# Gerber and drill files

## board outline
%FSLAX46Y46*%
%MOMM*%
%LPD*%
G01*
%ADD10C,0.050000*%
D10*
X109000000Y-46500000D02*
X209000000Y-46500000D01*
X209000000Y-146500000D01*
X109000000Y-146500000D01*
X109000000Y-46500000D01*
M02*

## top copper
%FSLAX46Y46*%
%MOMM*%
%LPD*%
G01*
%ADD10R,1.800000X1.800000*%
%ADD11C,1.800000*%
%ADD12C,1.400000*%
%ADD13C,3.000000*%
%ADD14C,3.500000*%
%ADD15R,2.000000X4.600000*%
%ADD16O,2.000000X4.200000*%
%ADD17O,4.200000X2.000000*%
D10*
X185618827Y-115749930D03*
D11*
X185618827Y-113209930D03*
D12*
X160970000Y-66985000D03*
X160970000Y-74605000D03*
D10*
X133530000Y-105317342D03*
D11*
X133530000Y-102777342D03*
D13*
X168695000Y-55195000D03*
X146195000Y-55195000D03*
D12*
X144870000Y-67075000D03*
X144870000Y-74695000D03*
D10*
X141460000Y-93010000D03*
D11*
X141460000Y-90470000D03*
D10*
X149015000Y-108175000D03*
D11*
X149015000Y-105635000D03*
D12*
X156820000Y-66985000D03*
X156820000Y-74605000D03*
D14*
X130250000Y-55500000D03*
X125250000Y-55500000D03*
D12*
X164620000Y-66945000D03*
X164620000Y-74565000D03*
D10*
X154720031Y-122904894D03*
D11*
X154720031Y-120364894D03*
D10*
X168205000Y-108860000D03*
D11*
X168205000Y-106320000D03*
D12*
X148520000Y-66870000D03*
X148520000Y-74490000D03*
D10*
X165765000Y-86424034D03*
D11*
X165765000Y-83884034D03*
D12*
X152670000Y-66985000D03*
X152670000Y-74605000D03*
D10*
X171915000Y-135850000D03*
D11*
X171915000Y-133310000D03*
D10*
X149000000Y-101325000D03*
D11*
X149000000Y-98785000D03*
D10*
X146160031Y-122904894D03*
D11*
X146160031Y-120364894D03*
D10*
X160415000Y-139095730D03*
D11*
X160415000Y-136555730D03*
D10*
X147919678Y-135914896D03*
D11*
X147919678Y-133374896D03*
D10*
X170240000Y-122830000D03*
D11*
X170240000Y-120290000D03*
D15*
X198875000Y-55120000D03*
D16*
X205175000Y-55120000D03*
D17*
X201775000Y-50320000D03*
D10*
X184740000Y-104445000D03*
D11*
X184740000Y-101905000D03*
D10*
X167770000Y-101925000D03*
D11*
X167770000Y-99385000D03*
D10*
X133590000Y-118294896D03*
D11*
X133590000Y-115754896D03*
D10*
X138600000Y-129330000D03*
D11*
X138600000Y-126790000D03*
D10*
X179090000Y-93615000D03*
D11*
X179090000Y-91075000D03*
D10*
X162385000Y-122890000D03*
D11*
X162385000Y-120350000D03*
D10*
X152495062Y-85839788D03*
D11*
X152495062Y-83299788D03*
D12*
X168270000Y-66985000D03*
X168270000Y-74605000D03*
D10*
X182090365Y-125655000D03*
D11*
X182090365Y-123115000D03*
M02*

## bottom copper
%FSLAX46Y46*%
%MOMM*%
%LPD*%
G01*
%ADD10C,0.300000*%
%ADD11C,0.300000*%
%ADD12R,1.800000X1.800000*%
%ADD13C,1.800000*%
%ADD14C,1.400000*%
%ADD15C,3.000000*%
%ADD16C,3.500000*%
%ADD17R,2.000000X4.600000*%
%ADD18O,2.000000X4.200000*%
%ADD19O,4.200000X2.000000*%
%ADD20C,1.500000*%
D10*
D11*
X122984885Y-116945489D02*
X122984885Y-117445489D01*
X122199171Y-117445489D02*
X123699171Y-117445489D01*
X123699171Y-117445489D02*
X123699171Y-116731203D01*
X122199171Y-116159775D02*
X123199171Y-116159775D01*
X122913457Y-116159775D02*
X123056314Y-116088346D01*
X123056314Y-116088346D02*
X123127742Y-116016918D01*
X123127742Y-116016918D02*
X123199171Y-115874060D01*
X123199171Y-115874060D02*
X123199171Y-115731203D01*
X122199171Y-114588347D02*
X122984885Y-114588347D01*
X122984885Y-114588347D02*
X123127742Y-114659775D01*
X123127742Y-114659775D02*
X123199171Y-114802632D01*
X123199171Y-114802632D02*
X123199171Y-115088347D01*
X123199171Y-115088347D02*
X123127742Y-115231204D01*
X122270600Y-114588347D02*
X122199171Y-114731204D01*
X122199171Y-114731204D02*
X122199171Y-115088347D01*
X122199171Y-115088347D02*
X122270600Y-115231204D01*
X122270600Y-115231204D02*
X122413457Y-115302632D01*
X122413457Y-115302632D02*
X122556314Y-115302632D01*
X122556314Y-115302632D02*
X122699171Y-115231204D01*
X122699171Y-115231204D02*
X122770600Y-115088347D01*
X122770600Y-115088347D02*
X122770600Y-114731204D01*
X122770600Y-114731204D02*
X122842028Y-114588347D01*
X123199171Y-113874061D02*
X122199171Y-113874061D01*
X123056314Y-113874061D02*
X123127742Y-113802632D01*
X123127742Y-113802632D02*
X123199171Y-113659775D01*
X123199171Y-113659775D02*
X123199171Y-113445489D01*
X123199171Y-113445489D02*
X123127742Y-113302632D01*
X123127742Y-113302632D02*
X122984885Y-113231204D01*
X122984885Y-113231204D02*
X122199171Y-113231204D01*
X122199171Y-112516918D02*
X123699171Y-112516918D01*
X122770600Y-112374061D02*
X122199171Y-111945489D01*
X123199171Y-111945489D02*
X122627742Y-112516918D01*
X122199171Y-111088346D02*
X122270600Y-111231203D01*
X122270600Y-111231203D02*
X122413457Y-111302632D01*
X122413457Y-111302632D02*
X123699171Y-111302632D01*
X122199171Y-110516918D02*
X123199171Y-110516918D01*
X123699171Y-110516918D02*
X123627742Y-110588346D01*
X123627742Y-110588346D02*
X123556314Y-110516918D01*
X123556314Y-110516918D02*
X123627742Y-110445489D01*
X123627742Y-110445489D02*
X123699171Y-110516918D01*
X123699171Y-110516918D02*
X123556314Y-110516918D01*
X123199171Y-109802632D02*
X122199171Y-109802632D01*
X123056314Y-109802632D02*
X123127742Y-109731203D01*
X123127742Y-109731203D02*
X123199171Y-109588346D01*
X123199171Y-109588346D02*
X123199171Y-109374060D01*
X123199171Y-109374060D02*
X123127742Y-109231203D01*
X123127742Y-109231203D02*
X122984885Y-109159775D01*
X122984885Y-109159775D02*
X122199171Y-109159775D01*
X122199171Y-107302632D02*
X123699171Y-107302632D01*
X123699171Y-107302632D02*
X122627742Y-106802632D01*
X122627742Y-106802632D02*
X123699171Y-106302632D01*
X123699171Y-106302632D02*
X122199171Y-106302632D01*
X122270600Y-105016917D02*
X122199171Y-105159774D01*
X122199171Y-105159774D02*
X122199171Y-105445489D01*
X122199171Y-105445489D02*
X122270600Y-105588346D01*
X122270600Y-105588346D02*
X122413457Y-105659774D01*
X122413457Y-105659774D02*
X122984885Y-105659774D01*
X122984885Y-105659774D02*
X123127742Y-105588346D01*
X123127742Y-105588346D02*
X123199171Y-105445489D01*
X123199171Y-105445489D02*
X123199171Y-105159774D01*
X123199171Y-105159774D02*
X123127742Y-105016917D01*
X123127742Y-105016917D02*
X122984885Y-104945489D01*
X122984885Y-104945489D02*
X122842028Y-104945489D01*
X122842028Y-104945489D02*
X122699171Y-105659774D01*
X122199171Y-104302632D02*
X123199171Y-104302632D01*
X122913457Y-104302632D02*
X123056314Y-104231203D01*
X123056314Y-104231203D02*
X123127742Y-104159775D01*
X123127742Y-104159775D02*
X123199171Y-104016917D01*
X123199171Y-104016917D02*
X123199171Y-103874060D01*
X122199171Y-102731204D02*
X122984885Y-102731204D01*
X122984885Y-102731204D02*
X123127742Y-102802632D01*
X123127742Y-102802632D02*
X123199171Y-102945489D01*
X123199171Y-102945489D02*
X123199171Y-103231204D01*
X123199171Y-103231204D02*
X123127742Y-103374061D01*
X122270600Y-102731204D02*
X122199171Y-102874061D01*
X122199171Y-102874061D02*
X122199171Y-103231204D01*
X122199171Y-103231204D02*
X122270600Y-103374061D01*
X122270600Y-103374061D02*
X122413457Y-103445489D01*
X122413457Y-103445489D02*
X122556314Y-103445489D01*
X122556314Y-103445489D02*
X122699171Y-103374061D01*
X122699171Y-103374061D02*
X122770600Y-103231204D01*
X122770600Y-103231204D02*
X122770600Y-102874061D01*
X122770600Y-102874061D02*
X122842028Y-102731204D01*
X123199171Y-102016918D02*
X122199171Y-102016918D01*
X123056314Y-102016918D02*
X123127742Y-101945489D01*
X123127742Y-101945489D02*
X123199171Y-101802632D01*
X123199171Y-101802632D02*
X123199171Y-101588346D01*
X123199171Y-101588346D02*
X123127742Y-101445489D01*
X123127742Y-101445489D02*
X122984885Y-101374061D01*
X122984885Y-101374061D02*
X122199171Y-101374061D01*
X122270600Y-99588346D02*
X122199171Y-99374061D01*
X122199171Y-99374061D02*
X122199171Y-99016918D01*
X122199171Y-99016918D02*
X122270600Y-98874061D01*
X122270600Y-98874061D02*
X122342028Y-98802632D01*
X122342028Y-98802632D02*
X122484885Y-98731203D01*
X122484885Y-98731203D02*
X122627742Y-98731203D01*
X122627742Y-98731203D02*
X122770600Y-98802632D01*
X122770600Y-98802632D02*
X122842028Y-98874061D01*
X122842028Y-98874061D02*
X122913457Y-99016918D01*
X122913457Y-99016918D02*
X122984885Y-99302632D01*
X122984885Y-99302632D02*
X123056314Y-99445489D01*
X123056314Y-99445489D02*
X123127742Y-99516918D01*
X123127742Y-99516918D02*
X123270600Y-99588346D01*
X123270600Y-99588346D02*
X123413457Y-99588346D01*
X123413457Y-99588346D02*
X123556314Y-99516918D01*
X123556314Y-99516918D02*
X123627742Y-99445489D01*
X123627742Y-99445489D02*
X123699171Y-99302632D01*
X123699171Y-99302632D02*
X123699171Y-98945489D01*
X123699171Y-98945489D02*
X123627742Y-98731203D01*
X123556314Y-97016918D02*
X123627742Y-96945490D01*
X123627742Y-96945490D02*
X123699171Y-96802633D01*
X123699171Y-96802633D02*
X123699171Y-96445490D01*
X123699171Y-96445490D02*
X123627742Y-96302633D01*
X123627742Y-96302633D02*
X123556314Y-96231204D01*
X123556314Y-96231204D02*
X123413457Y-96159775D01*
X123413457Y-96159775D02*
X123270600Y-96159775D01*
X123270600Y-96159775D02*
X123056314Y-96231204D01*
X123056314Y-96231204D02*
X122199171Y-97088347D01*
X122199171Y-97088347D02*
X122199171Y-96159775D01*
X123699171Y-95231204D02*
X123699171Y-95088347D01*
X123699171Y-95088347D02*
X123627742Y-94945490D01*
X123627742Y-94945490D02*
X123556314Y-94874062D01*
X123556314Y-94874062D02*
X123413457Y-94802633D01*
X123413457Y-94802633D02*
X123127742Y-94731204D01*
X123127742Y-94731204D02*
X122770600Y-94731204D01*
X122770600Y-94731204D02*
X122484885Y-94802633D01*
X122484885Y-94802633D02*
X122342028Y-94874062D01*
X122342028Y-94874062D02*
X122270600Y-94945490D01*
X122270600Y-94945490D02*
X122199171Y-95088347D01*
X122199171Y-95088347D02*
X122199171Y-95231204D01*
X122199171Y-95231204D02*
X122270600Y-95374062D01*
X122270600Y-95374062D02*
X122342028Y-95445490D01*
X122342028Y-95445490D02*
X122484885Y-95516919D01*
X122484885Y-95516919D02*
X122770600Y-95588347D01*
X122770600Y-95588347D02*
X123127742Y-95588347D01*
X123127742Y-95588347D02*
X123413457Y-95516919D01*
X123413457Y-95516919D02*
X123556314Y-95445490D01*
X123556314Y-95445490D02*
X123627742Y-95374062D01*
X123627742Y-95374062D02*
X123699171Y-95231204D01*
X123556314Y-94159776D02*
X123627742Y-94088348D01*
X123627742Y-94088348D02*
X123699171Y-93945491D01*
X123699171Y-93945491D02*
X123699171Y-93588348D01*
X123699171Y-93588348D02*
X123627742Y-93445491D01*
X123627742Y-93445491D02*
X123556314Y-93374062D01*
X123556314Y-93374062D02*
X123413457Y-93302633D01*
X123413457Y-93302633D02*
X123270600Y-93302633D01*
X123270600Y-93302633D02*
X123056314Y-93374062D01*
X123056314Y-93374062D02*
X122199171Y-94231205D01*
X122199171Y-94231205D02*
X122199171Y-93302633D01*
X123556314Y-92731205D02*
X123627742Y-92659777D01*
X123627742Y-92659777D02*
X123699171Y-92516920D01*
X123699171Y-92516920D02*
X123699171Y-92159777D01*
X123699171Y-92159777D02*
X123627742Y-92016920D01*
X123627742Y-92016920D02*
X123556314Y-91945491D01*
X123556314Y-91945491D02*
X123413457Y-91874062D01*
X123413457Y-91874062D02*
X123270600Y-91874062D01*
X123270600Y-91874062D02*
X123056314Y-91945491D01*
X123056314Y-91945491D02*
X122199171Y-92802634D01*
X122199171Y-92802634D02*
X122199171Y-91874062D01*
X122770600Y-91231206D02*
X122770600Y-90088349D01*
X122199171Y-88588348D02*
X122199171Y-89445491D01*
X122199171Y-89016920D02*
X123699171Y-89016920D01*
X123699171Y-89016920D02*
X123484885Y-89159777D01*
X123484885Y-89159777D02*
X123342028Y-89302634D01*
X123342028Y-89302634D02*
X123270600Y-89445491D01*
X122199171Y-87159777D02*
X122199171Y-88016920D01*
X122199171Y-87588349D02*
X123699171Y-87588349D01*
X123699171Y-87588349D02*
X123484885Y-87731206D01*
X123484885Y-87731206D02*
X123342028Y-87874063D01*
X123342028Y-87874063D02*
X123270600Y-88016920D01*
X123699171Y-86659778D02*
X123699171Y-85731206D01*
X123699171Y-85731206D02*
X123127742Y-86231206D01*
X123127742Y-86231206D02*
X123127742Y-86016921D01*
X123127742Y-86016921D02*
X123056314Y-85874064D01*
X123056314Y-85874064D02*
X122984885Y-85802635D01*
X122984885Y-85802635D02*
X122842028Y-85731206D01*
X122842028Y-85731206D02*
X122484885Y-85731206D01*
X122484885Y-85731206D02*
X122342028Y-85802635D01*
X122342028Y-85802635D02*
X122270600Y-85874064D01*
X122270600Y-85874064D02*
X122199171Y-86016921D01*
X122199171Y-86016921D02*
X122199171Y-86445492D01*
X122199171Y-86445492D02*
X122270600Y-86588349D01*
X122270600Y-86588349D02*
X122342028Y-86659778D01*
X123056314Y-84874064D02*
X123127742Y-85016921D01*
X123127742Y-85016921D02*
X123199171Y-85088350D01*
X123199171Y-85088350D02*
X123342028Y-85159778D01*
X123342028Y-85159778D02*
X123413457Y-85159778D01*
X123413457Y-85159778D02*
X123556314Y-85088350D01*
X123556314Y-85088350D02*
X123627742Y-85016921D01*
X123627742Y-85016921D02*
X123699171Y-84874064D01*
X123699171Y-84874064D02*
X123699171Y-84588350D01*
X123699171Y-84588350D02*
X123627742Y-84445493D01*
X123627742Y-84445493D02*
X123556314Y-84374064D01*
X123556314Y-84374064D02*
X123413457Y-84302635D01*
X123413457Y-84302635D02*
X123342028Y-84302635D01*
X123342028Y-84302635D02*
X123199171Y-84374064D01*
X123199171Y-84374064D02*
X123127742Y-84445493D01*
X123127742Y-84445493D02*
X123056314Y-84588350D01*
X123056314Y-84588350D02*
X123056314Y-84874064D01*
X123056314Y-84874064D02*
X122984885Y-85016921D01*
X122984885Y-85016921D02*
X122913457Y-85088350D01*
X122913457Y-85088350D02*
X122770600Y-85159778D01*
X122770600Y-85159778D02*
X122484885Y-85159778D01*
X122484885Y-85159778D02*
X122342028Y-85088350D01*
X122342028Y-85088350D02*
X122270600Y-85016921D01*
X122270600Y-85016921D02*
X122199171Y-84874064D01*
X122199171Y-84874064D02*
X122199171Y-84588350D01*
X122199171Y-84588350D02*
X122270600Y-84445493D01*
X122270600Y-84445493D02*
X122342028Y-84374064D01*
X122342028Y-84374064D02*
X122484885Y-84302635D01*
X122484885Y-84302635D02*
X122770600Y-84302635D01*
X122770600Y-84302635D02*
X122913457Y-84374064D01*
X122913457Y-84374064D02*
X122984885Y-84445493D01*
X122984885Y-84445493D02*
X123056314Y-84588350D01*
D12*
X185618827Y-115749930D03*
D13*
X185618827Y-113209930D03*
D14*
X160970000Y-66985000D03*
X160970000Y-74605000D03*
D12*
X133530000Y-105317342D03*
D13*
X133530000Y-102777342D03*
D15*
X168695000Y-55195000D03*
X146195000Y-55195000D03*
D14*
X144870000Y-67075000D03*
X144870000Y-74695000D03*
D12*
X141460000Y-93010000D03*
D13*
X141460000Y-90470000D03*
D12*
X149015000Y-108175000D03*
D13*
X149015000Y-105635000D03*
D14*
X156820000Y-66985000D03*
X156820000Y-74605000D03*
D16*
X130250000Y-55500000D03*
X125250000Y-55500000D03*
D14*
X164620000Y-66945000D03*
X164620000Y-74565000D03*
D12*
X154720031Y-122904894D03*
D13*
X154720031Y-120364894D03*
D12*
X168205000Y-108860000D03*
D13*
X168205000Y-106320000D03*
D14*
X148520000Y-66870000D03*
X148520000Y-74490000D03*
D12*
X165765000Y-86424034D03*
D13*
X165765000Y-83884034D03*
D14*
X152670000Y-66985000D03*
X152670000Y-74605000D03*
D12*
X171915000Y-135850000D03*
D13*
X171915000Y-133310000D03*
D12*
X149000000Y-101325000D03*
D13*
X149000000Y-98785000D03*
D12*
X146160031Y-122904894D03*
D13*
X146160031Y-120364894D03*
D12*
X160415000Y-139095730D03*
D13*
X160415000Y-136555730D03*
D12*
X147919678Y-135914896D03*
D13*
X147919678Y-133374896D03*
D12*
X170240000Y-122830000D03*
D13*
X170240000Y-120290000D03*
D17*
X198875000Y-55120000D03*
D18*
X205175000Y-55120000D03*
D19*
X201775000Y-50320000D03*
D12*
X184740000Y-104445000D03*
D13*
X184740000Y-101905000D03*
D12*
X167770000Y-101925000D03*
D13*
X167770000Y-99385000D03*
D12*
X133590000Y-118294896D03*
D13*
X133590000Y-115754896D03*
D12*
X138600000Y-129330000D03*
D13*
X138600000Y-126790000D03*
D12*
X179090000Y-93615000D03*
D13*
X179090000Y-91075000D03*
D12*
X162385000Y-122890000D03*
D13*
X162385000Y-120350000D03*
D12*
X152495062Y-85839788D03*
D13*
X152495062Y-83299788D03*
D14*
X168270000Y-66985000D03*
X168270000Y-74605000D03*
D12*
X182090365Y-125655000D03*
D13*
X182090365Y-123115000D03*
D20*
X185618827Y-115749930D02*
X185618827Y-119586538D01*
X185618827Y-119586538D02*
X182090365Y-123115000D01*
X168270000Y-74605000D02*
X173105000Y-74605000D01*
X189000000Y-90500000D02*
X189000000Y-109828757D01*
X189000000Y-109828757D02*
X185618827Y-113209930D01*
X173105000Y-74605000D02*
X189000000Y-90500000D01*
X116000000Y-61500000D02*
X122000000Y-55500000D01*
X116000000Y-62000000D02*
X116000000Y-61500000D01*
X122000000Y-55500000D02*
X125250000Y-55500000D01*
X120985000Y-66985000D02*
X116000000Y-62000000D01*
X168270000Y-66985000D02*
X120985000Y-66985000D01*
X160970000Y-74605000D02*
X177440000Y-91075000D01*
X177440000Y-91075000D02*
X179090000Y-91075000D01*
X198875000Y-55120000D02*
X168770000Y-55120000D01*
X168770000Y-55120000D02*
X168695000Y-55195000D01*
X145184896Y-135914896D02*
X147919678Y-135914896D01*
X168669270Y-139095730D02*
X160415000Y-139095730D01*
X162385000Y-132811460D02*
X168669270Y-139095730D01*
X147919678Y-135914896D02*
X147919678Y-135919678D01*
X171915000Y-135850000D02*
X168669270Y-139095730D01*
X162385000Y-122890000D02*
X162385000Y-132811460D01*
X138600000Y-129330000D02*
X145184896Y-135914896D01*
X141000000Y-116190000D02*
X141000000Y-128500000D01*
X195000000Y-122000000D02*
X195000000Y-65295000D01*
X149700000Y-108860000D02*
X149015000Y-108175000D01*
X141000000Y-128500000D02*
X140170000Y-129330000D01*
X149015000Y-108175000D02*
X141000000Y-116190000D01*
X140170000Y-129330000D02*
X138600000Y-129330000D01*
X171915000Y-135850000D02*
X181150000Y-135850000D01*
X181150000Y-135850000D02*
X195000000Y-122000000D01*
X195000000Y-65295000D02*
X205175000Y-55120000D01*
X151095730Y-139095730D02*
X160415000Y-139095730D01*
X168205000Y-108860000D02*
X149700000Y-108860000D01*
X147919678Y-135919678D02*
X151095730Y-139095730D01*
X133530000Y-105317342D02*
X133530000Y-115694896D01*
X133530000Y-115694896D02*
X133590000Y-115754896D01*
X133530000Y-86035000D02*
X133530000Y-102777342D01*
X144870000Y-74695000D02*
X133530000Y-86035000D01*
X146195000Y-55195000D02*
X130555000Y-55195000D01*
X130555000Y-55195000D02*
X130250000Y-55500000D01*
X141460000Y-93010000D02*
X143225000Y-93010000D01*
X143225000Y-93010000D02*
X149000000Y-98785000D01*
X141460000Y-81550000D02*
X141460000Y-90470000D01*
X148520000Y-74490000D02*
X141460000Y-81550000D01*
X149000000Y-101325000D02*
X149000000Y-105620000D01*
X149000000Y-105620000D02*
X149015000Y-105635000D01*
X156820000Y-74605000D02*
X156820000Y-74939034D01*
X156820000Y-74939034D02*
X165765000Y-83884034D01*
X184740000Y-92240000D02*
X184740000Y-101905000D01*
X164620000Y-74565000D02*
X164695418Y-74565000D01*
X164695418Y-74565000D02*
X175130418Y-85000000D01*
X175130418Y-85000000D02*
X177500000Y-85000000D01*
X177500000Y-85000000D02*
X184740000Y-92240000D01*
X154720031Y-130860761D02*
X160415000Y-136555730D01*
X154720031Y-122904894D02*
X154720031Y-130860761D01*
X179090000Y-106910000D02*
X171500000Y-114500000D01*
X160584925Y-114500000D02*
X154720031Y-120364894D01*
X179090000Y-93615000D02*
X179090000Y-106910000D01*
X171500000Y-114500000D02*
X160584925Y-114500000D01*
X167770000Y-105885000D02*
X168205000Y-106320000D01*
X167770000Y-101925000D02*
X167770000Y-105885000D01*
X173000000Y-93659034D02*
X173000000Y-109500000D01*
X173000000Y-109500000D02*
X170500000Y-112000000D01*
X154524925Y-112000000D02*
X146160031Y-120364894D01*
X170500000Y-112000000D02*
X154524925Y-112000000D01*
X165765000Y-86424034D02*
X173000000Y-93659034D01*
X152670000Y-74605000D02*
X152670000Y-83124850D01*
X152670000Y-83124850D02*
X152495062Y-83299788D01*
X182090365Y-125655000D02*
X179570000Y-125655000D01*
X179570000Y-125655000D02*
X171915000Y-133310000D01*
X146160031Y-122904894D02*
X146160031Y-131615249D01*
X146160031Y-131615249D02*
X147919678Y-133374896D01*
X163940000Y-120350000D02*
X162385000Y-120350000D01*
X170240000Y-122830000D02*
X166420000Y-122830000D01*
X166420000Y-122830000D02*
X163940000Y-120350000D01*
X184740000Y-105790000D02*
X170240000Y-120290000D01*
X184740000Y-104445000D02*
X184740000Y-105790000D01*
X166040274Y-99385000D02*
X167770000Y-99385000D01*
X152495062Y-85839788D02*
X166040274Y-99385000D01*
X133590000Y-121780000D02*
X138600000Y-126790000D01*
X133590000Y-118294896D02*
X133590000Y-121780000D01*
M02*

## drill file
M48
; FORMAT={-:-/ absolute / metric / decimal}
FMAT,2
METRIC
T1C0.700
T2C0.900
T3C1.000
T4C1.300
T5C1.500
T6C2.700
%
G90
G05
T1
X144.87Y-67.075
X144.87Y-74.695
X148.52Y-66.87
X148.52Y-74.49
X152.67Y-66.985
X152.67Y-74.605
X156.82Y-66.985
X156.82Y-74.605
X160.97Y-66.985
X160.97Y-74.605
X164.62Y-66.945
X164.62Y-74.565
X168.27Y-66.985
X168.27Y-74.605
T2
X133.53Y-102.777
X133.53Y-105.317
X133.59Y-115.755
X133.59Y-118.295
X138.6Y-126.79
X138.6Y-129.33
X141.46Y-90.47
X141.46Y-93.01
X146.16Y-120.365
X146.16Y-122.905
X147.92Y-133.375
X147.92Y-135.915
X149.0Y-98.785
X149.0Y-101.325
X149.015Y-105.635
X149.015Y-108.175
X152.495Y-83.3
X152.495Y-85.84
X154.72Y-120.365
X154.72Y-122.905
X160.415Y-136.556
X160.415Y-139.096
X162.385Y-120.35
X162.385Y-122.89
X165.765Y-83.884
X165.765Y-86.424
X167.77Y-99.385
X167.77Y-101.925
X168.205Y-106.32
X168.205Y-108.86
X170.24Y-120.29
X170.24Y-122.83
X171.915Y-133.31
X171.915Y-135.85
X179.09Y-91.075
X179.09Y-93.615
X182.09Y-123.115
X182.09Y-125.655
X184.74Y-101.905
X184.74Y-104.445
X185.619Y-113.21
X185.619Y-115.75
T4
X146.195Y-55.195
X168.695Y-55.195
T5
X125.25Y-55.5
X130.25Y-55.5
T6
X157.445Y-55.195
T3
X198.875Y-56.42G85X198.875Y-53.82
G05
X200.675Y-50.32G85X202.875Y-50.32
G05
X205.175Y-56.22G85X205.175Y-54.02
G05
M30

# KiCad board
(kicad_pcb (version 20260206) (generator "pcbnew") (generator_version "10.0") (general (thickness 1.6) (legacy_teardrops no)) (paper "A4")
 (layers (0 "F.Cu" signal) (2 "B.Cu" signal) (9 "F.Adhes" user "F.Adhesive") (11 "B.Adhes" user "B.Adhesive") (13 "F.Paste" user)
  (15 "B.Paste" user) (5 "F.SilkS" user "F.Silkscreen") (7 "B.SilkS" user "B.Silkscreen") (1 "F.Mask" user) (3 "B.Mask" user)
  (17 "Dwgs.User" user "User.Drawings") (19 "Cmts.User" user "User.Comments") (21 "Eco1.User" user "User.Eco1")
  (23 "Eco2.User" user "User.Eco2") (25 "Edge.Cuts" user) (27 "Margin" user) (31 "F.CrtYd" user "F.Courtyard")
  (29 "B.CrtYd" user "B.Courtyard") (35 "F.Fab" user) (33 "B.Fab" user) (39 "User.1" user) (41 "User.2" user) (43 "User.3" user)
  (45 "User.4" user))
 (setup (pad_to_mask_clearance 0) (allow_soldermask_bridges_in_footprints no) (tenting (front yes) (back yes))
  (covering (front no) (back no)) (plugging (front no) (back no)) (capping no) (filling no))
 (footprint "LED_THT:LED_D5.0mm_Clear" (layer "F.Cu") (at 185.618827 115.74993 90)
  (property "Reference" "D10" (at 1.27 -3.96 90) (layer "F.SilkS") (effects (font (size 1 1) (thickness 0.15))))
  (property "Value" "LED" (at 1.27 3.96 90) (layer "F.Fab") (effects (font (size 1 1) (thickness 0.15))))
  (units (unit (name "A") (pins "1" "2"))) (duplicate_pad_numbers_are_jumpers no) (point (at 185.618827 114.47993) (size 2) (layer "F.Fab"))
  (pad "1" thru_hole rect (at 0 0 90) (size 1.8 1.8) (drill 0.9) (layers "*.Cu" "*.Mask") (remove_unused_layers no) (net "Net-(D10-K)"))
  (pad "2" thru_hole circle (at 2.54 0 90) (size 1.8 1.8) (drill 0.9) (layers "*.Cu" "*.Mask") (remove_unused_layers no) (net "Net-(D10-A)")))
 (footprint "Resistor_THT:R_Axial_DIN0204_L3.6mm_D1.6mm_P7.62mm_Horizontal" (layer "F.Cu") (at 160.97 66.985 -90)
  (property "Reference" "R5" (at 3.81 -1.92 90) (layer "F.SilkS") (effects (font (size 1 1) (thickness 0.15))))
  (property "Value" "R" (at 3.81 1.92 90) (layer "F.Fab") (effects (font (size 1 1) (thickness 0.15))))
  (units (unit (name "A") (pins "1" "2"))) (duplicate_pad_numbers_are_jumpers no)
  (pad "1" thru_hole circle (at 0 0 270) (size 1.4 1.4) (drill 0.7) (layers "*.Cu" "*.Mask") (remove_unused_layers no) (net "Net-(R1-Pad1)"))
  (pad "2" thru_hole circle (at 7.62 0 270) (size 1.4 1.4) (drill 0.7) (layers "*.Cu" "*.Mask") (remove_unused_layers no)
   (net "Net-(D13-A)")))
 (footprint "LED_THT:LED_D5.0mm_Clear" (layer "F.Cu") (at 133.53 105.317342 90)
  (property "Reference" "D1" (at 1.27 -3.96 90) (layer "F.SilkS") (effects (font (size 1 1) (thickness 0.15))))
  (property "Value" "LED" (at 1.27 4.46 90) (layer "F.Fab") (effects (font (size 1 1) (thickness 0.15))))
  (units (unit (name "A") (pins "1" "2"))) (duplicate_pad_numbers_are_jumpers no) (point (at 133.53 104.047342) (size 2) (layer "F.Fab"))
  (pad "1" thru_hole rect (at 0 0 90) (size 1.8 1.8) (drill 0.9) (layers "*.Cu" "*.Mask") (remove_unused_layers no) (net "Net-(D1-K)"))
  (pad "2" thru_hole circle (at 2.54 0 90) (size 1.8 1.8) (drill 0.9) (layers "*.Cu" "*.Mask") (remove_unused_layers no) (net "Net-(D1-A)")))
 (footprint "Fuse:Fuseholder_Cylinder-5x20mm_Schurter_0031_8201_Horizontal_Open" (layer "F.Cu") (at 168.695 55.195 180)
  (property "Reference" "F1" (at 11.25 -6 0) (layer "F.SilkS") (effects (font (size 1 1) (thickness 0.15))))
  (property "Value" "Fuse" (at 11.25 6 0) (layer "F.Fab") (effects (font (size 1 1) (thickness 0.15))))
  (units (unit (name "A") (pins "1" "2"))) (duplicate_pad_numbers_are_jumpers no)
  (pad "" np_thru_hole circle (at 11.25 0 180) (size 2.7 2.7) (drill 2.7) (layers "*.Cu" "*.Mask"))
  (pad "1" thru_hole circle (at 0 0 180) (size 3 3) (drill 1.3) (layers "*.Cu" "*.Mask") (remove_unused_layers no) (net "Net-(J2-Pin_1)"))
  (pad "2" thru_hole circle (at 22.5 0 180) (size 3 3) (drill 1.3) (layers "*.Cu" "*.Mask") (remove_unused_layers no) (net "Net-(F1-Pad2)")))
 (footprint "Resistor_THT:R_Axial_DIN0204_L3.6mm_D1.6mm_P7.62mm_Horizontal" (layer "F.Cu") (at 144.87 67.075 -90)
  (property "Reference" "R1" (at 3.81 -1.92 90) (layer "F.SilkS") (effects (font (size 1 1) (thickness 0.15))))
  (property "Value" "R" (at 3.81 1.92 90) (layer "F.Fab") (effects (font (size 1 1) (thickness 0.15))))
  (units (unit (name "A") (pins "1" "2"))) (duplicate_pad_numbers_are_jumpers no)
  (pad "1" thru_hole circle (at 0 0 270) (size 1.4 1.4) (drill 0.7) (layers "*.Cu" "*.Mask") (remove_unused_layers no) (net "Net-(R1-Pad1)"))
  (pad "2" thru_hole circle (at 7.62 0 270) (size 1.4 1.4) (drill 0.7) (layers "*.Cu" "*.Mask") (remove_unused_layers no) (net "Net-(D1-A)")))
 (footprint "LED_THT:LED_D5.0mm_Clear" (layer "F.Cu") (at 141.46 93.01 90)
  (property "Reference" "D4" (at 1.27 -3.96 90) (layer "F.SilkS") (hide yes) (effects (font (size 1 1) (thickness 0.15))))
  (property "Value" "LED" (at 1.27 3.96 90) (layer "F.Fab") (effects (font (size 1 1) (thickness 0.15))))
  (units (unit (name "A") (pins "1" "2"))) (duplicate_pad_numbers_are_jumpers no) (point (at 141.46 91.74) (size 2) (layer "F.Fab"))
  (pad "1" thru_hole rect (at 0 0 90) (size 1.8 1.8) (drill 0.9) (layers "*.Cu" "*.Mask") (remove_unused_layers no) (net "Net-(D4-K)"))
  (pad "2" thru_hole circle (at 2.54 0 90) (size 1.8 1.8) (drill 0.9) (layers "*.Cu" "*.Mask") (remove_unused_layers no) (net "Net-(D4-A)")))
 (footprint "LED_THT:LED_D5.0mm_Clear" (layer "F.Cu") (at 149.015 108.175 90)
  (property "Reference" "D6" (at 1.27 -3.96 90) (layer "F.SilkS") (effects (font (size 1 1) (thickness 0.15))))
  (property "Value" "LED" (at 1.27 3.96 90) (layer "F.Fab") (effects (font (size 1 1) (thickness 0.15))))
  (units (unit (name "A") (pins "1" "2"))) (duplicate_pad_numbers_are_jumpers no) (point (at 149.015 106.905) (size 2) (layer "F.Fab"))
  (pad "1" thru_hole rect (at 0 0 90) (size 1.8 1.8) (drill 0.9) (layers "*.Cu" "*.Mask") (remove_unused_layers no) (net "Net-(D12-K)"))
  (pad "2" thru_hole circle (at 2.54 0 90) (size 1.8 1.8) (drill 0.9) (layers "*.Cu" "*.Mask") (remove_unused_layers no) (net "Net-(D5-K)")))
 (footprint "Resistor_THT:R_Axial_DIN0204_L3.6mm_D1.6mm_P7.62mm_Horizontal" (layer "F.Cu") (at 156.82 66.985 -90)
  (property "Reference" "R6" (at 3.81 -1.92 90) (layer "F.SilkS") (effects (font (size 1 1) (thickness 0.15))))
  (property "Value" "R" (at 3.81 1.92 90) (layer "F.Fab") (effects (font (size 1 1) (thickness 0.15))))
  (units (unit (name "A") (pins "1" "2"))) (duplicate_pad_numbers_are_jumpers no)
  (pad "1" thru_hole circle (at 0 0 270) (size 1.4 1.4) (drill 0.7) (layers "*.Cu" "*.Mask") (remove_unused_layers no) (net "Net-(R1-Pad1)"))
  (pad "2" thru_hole circle (at 7.62 0 270) (size 1.4 1.4) (drill 0.7) (layers "*.Cu" "*.Mask") (remove_unused_layers no)
   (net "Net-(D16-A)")))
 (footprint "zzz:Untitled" (layer "F.Cu") (at 125.25 50.5 180)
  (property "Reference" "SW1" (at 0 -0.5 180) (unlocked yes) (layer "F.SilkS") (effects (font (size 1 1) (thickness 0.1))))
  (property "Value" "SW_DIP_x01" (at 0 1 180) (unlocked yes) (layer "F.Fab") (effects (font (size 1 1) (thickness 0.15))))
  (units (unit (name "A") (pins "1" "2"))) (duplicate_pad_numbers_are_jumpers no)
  (pad "1" thru_hole circle (at -5 -5 180) (size 3.5 3.5) (drill 1.5) (layers "*.Cu" "*.Mask") (remove_unused_layers no)
   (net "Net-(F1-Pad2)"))
  (pad "2" thru_hole circle (at 0 -5 180) (size 3.5 3.5) (drill 1.5) (layers "*.Cu" "*.Mask") (remove_unused_layers no)
   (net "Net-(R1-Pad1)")))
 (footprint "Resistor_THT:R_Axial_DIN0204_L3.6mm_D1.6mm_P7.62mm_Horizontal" (layer "F.Cu") (at 164.62 66.945 -90)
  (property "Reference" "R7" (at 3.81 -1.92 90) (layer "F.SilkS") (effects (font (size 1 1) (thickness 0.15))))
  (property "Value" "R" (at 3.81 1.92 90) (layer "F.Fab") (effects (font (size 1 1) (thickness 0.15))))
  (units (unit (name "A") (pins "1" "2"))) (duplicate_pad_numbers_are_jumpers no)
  (pad "1" thru_hole circle (at 0 0 270) (size 1.4 1.4) (drill 0.7) (layers "*.Cu" "*.Mask") (remove_unused_layers no) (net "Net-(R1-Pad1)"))
  (pad "2" thru_hole circle (at 7.62 0 270) (size 1.4 1.4) (drill 0.7) (layers "*.Cu" "*.Mask") (remove_unused_layers no)
   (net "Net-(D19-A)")))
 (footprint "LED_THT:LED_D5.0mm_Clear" (layer "F.Cu") (at 154.720031 122.904894 90)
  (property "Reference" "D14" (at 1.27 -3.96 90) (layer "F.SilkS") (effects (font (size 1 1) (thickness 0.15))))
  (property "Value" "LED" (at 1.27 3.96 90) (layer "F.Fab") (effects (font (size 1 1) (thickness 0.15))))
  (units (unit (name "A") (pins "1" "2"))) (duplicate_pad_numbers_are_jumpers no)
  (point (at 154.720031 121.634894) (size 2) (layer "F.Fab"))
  (pad "1" thru_hole rect (at 0 0 90) (size 1.8 1.8) (drill 0.9) (layers "*.Cu" "*.Mask") (remove_unused_layers no) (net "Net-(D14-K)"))
  (pad "2" thru_hole circle (at 2.54 0 90) (size 1.8 1.8) (drill 0.9) (layers "*.Cu" "*.Mask") (remove_unused_layers no) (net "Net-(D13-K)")))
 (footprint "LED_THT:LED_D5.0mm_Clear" (layer "F.Cu") (at 168.205 108.86 90)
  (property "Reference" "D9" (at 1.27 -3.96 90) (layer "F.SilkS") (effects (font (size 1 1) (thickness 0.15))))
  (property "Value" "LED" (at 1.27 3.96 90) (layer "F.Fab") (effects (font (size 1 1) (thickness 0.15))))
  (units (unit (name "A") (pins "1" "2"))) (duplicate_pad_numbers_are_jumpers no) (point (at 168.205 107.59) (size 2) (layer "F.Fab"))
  (pad "1" thru_hole rect (at 0 0 90) (size 1.8 1.8) (drill 0.9) (layers "*.Cu" "*.Mask") (remove_unused_layers no) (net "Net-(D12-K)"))
  (pad "2" thru_hole circle (at 2.54 0 90) (size 1.8 1.8) (drill 0.9) (layers "*.Cu" "*.Mask") (remove_unused_layers no) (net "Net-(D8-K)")))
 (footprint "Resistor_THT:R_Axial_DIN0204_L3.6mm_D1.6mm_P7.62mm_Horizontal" (layer "F.Cu") (at 148.52 66.87 -90)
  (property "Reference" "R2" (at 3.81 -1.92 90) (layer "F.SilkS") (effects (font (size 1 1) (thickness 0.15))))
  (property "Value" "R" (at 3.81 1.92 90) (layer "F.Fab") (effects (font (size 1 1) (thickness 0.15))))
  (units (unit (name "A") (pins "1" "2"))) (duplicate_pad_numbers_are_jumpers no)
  (pad "1" thru_hole circle (at 0 0 270) (size 1.4 1.4) (drill 0.7) (layers "*.Cu" "*.Mask") (remove_unused_layers no) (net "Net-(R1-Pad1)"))
  (pad "2" thru_hole circle (at 7.62 0 270) (size 1.4 1.4) (drill 0.7) (layers "*.Cu" "*.Mask") (remove_unused_layers no) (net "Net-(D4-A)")))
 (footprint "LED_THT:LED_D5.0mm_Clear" (layer "F.Cu") (at 165.765 86.424034 90)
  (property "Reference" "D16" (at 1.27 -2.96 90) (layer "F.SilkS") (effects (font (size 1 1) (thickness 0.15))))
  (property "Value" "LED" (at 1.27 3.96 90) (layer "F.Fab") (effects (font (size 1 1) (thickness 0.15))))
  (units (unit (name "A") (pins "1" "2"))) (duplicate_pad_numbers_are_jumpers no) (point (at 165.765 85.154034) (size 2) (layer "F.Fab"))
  (pad "1" thru_hole rect (at 0 0 90) (size 1.8 1.8) (drill 0.9) (layers "*.Cu" "*.Mask") (remove_unused_layers no) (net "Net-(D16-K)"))
  (pad "2" thru_hole circle (at 2.54 0 90) (size 1.8 1.8) (drill 0.9) (layers "*.Cu" "*.Mask") (remove_unused_layers no) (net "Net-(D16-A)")))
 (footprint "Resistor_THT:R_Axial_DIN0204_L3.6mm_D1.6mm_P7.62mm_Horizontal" (layer "F.Cu") (at 152.67 66.985 -90)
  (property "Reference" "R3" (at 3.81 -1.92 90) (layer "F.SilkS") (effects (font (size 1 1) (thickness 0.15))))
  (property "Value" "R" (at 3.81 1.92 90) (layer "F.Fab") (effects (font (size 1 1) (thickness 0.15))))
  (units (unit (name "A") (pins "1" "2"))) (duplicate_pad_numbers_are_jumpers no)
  (pad "1" thru_hole circle (at 0 0 270) (size 1.4 1.4) (drill 0.7) (layers "*.Cu" "*.Mask") (remove_unused_layers no) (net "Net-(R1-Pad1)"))
  (pad "2" thru_hole circle (at 7.62 0 270) (size 1.4 1.4) (drill 0.7) (layers "*.Cu" "*.Mask") (remove_unused_layers no) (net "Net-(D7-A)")))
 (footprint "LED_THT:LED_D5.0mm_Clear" (layer "F.Cu") (at 171.915 135.85 90)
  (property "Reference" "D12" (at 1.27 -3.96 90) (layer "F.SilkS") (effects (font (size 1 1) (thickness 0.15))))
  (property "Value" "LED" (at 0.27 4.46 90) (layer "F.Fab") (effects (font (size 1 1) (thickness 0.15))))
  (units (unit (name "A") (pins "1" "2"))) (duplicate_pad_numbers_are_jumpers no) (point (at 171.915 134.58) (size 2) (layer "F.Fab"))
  (pad "1" thru_hole rect (at 0 0 90) (size 1.8 1.8) (drill 0.9) (layers "*.Cu" "*.Mask") (remove_unused_layers no) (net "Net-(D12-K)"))
  (pad "2" thru_hole circle (at 2.54 0 90) (size 1.8 1.8) (drill 0.9) (layers "*.Cu" "*.Mask") (remove_unused_layers no) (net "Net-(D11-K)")))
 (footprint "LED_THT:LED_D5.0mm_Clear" (layer "F.Cu") (at 149 101.325 90)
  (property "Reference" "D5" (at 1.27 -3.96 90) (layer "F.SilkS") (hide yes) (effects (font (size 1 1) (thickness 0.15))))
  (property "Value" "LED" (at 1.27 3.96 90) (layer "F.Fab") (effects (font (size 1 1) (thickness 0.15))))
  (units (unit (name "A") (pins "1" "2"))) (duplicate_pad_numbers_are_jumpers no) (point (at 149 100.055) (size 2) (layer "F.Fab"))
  (pad "1" thru_hole rect (at 0 0 90) (size 1.8 1.8) (drill 0.9) (layers "*.Cu" "*.Mask") (remove_unused_layers no) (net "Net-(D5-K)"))
  (pad "2" thru_hole circle (at 2.54 0 90) (size 1.8 1.8) (drill 0.9) (layers "*.Cu" "*.Mask") (remove_unused_layers no) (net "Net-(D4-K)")))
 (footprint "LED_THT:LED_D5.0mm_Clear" (layer "F.Cu") (at 146.160031 122.904894 90)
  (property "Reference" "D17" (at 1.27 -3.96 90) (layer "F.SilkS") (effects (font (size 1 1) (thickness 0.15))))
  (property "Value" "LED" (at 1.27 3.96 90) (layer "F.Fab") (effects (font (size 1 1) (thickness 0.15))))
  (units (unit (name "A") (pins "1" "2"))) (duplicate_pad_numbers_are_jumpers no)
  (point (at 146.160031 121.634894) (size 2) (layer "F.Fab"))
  (pad "1" thru_hole rect (at 0 0 90) (size 1.8 1.8) (drill 0.9) (layers "*.Cu" "*.Mask") (remove_unused_layers no) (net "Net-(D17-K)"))
  (pad "2" thru_hole circle (at 2.54 0 90) (size 1.8 1.8) (drill 0.9) (layers "*.Cu" "*.Mask") (remove_unused_layers no) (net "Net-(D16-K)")))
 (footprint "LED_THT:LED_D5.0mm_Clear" (layer "F.Cu") (at 160.415 139.09573 90)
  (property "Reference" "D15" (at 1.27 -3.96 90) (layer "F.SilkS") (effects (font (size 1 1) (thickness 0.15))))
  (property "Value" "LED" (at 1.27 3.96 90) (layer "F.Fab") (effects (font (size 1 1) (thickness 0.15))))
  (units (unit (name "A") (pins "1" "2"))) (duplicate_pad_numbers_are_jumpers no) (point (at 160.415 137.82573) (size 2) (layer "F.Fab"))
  (pad "1" thru_hole rect (at 0 0 90) (size 1.8 1.8) (drill 0.9) (layers "*.Cu" "*.Mask") (remove_unused_layers no) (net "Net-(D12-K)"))
  (pad "2" thru_hole circle (at 2.54 0 90) (size 1.8 1.8) (drill 0.9) (layers "*.Cu" "*.Mask") (remove_unused_layers no) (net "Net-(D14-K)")))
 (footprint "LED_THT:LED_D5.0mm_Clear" (layer "F.Cu") (at 147.919678 135.914896 90)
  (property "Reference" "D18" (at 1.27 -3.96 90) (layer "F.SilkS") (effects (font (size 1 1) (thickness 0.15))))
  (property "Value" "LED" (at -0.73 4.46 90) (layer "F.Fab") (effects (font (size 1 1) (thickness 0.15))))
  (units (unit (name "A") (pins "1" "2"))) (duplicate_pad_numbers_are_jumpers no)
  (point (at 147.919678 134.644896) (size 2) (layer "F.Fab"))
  (pad "1" thru_hole rect (at 0 0 90) (size 1.8 1.8) (drill 0.9) (layers "*.Cu" "*.Mask") (remove_unused_layers no) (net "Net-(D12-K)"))
  (pad "2" thru_hole circle (at 2.54 0 90) (size 1.8 1.8) (drill 0.9) (layers "*.Cu" "*.Mask") (remove_unused_layers no) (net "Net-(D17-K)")))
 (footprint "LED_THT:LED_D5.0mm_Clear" (layer "F.Cu") (at 170.24 122.83 90)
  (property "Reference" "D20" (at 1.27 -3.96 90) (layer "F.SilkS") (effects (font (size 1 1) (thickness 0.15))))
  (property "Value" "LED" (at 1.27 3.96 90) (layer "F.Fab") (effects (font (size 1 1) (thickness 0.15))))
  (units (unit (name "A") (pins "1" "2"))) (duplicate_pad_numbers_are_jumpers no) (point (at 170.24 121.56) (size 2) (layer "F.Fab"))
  (pad "1" thru_hole rect (at 0 0 90) (size 1.8 1.8) (drill 0.9) (layers "*.Cu" "*.Mask") (remove_unused_layers no) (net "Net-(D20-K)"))
  (pad "2" thru_hole circle (at 2.54 0 90) (size 1.8 1.8) (drill 0.9) (layers "*.Cu" "*.Mask") (remove_unused_layers no) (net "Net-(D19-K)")))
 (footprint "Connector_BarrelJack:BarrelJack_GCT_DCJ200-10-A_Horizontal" (layer "F.Cu") (at 198.875 55.12 90)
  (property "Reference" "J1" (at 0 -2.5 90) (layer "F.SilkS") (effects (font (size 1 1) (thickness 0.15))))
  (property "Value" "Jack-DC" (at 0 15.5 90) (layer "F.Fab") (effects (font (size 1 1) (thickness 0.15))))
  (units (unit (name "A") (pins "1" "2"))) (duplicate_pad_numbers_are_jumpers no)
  (pad "1" thru_hole rect (at 0 0 90) (size 4.6 2) (drill oval 3.6 1) (layers "*.Cu" "*.Mask") (remove_unused_layers no)
   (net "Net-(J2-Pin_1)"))
  (pad "2" thru_hole oval (at 0 6.3 90) (size 4.2 2) (drill oval 3.2 1) (layers "*.Cu" "*.Mask") (remove_unused_layers no)
   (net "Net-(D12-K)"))
  (pad "3" thru_hole oval (at 4.8 2.9 90) (size 2 4.2) (drill oval 1 3.2) (layers "*.Cu" "*.Mask") (remove_unused_layers no)))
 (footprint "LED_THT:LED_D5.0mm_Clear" (layer "F.Cu") (at 184.74 104.445 90)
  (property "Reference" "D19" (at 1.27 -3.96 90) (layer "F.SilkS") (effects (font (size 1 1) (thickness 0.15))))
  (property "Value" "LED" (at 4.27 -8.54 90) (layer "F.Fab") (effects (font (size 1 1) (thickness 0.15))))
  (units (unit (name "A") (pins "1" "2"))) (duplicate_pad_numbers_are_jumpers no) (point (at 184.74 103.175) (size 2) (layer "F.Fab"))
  (pad "1" thru_hole rect (at 0 0 90) (size 1.8 1.8) (drill 0.9) (layers "*.Cu" "*.Mask") (remove_unused_layers no) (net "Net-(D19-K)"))
  (pad "2" thru_hole circle (at 2.54 0 90) (size 1.8 1.8) (drill 0.9) (layers "*.Cu" "*.Mask") (remove_unused_layers no) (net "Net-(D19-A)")))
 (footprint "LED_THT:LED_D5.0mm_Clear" (layer "F.Cu") (at 167.77 101.925 90)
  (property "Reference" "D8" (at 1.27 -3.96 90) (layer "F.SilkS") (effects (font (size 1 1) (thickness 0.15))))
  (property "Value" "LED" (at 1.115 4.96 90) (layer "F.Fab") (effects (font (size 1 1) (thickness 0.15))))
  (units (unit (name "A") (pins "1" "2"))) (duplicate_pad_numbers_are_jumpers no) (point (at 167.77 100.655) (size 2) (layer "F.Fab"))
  (pad "1" thru_hole rect (at 0 0 90) (size 1.8 1.8) (drill 0.9) (layers "*.Cu" "*.Mask") (remove_unused_layers no) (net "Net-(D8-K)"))
  (pad "2" thru_hole circle (at 2.54 0 90) (size 1.8 1.8) (drill 0.9) (layers "*.Cu" "*.Mask") (remove_unused_layers no) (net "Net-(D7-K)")))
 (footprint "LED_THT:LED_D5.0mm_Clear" (layer "F.Cu") (at 133.59 118.294896 90)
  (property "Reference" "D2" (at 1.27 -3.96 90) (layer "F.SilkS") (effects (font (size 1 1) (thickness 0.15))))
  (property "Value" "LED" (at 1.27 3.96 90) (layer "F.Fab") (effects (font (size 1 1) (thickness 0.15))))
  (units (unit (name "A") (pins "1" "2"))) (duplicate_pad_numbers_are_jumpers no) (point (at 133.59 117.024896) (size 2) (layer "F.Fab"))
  (pad "1" thru_hole rect (at 0 0 90) (size 1.8 1.8) (drill 0.9) (layers "*.Cu" "*.Mask") (remove_unused_layers no) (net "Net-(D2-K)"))
  (pad "2" thru_hole circle (at 2.54 0 90) (size 1.8 1.8) (drill 0.9) (layers "*.Cu" "*.Mask") (remove_unused_layers no) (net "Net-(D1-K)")))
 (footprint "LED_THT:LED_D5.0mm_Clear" (layer "F.Cu") (at 138.6 129.33 90)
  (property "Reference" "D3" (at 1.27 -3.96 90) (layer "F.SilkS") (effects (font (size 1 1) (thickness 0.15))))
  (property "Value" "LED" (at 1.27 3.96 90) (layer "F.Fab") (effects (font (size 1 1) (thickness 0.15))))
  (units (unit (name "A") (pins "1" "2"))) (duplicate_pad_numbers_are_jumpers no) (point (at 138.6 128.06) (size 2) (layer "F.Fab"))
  (pad "1" thru_hole rect (at 0 0 90) (size 1.8 1.8) (drill 0.9) (layers "*.Cu" "*.Mask") (remove_unused_layers no) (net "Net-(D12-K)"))
  (pad "2" thru_hole circle (at 2.54 0 90) (size 1.8 1.8) (drill 0.9) (layers "*.Cu" "*.Mask") (remove_unused_layers no) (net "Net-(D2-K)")))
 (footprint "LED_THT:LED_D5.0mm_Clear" (layer "F.Cu") (at 179.09 93.615 90)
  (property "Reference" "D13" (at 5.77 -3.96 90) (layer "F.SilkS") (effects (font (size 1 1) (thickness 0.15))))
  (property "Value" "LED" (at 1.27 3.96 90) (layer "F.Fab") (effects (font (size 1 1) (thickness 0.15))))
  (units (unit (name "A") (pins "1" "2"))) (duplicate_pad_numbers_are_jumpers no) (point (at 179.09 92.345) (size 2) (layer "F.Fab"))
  (pad "1" thru_hole rect (at 0 0 90) (size 1.8 1.8) (drill 0.9) (layers "*.Cu" "*.Mask") (remove_unused_layers no) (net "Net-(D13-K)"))
  (pad "2" thru_hole circle (at 2.54 0 90) (size 1.8 1.8) (drill 0.9) (layers "*.Cu" "*.Mask") (remove_unused_layers no) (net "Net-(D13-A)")))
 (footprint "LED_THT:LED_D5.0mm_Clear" (layer "F.Cu") (at 162.385 122.89 90)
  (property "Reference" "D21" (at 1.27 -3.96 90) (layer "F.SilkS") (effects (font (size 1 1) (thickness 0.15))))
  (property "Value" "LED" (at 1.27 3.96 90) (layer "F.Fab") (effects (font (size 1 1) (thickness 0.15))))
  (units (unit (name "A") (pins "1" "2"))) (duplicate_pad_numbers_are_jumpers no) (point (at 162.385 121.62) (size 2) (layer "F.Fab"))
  (pad "1" thru_hole rect (at 0 0 90) (size 1.8 1.8) (drill 0.9) (layers "*.Cu" "*.Mask") (remove_unused_layers no) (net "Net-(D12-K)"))
  (pad "2" thru_hole circle (at 2.54 0 90) (size 1.8 1.8) (drill 0.9) (layers "*.Cu" "*.Mask") (remove_unused_layers no) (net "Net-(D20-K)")))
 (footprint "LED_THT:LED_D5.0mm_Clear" (layer "F.Cu") (at 152.495062 85.839788 90)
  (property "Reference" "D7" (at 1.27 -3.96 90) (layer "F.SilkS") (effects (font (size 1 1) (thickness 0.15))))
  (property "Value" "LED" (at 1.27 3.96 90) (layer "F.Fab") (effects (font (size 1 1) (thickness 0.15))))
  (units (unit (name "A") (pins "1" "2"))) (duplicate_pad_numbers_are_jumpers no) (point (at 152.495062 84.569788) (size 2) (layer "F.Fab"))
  (pad "1" thru_hole rect (at 0 0 90) (size 1.8 1.8) (drill 0.9) (layers "*.Cu" "*.Mask") (remove_unused_layers no) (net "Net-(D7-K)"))
  (pad "2" thru_hole circle (at 2.54 0 90) (size 1.8 1.8) (drill 0.9) (layers "*.Cu" "*.Mask") (remove_unused_layers no) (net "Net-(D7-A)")))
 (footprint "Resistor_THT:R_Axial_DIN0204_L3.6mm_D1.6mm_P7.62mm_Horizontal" (layer "F.Cu") (at 168.27 66.985 -90)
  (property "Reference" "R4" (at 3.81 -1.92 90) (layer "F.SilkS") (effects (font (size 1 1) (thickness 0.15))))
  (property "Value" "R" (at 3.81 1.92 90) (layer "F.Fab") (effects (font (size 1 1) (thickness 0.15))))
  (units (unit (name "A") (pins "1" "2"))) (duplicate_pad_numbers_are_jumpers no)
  (pad "1" thru_hole circle (at 0 0 270) (size 1.4 1.4) (drill 0.7) (layers "*.Cu" "*.Mask") (remove_unused_layers no) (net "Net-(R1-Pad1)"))
  (pad "2" thru_hole circle (at 7.62 0 270) (size 1.4 1.4) (drill 0.7) (layers "*.Cu" "*.Mask") (remove_unused_layers no)
   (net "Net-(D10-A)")))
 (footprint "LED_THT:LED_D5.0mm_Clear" (layer "F.Cu") (at 182.090365 125.655 90)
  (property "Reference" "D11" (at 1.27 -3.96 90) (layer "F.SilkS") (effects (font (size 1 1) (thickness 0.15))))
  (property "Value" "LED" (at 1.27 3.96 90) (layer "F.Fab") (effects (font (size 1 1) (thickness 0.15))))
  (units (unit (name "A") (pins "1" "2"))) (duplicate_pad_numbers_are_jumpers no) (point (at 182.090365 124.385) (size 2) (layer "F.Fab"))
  (pad "1" thru_hole rect (at 0 0 90) (size 1.8 1.8) (drill 0.9) (layers "*.Cu" "*.Mask") (remove_unused_layers no) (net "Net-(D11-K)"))
  (pad "2" thru_hole circle (at 2.54 0 90) (size 1.8 1.8) (drill 0.9) (layers "*.Cu" "*.Mask") (remove_unused_layers no) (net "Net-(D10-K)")))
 (gr_rect (start 109 46.5) (end 209 146.5) (stroke (width 0.05) (type default)) (fill no) (layer "Edge.Cuts"))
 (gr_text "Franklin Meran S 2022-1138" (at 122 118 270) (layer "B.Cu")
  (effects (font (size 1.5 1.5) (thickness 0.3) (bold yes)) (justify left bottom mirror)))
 (segment (start 185.618827 115.74993) (end 185.618827 119.586538) (width 1.5) (layer "B.Cu") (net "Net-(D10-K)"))
 (segment (start 185.618827 119.586538) (end 182.090365 123.115) (width 1.5) (layer "B.Cu") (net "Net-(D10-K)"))
 (segment (start 168.27 74.605) (end 173.105 74.605) (width 1.5) (layer "B.Cu") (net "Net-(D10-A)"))
 (segment (start 189 90.5) (end 189 109.828757) (width 1.5) (layer "B.Cu") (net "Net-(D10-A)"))
 (segment (start 189 109.828757) (end 185.618827 113.20993) (width 1.5) (layer "B.Cu") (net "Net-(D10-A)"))
 (segment (start 173.105 74.605) (end 189 90.5) (width 1.5) (layer "B.Cu") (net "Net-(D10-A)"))
 (segment (start 116 61.5) (end 122 55.5) (width 1.5) (layer "B.Cu") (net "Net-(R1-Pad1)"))
 (segment (start 116 62) (end 116 61.5) (width 1.5) (layer "B.Cu") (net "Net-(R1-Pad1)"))
 (segment (start 122 55.5) (end 125.25 55.5) (width 1.5) (layer "B.Cu") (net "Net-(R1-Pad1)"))
 (segment (start 120.985 66.985) (end 116 62) (width 1.5) (layer "B.Cu") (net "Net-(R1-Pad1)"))
 (segment (start 168.27 66.985) (end 120.985 66.985) (width 1.5) (layer "B.Cu") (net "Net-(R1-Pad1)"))
 (segment (start 160.97 74.605) (end 177.44 91.075) (width 1.5) (layer "B.Cu") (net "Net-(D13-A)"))
 (segment (start 177.44 91.075) (end 179.09 91.075) (width 1.5) (layer "B.Cu") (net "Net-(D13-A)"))
 (segment (start 198.875 55.12) (end 168.77 55.12) (width 1.5) (layer "B.Cu") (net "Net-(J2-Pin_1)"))
 (segment (start 168.77 55.12) (end 168.695 55.195) (width 1.5) (layer "B.Cu") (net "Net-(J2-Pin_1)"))
 (segment (start 145.184896 135.914896) (end 147.919678 135.914896) (width 1.5) (layer "B.Cu") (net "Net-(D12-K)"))
 (segment (start 168.66927 139.09573) (end 160.415 139.09573) (width 1.5) (layer "B.Cu") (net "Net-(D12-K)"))
 (segment (start 162.385 132.81146) (end 168.66927 139.09573) (width 1.5) (layer "B.Cu") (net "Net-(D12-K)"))
 (segment (start 147.919678 135.914896) (end 147.919678 135.919678) (width 1.5) (layer "B.Cu") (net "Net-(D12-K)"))
 (segment (start 171.915 135.85) (end 168.66927 139.09573) (width 1.5) (layer "B.Cu") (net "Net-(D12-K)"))
 (segment (start 162.385 122.89) (end 162.385 132.81146) (width 1.5) (layer "B.Cu") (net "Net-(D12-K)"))
 (segment (start 138.6 129.33) (end 145.184896 135.914896) (width 1.5) (layer "B.Cu") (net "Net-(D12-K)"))
 (segment (start 141 116.19) (end 141 128.5) (width 1.5) (layer "B.Cu") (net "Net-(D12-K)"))
 (segment (start 195 122) (end 195 65.295) (width 1.5) (layer "B.Cu") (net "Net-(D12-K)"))
 (segment (start 149.7 108.86) (end 149.015 108.175) (width 1.5) (layer "B.Cu") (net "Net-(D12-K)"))
 (segment (start 141 128.5) (end 140.17 129.33) (width 1.5) (layer "B.Cu") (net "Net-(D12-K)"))
 (segment (start 149.015 108.175) (end 141 116.19) (width 1.5) (layer "B.Cu") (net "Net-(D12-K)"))
 (segment (start 140.17 129.33) (end 138.6 129.33) (width 1.5) (layer "B.Cu") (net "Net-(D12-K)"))
 (segment (start 171.915 135.85) (end 181.15 135.85) (width 1.5) (layer "B.Cu") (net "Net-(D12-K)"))
 (segment (start 181.15 135.85) (end 195 122) (width 1.5) (layer "B.Cu") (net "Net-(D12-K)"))
 (segment (start 195 65.295) (end 205.175 55.12) (width 1.5) (layer "B.Cu") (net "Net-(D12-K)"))
 (segment (start 151.09573 139.09573) (end 160.415 139.09573) (width 1.5) (layer "B.Cu") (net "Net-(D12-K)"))
 (segment (start 168.205 108.86) (end 149.7 108.86) (width 1.5) (layer "B.Cu") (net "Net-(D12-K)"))
 (segment (start 147.919678 135.919678) (end 151.09573 139.09573) (width 1.5) (layer "B.Cu") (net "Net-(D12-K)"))
 (segment (start 133.53 105.317342) (end 133.53 115.694896) (width 1.5) (layer "B.Cu") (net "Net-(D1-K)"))
 (segment (start 133.53 115.694896) (end 133.59 115.754896) (width 1.5) (layer "B.Cu") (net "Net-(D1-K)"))
 (segment (start 133.53 86.035) (end 133.53 102.777342) (width 1.5) (layer "B.Cu") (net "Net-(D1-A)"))
 (segment (start 144.87 74.695) (end 133.53 86.035) (width 1.5) (layer "B.Cu") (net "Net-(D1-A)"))
 (segment (start 146.195 55.195) (end 130.555 55.195) (width 1.5) (layer "B.Cu") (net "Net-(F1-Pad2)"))
 (segment (start 130.555 55.195) (end 130.25 55.5) (width 1.5) (layer "B.Cu") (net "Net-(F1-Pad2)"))
 (segment (start 141.46 93.01) (end 143.225 93.01) (width 1.5) (layer "B.Cu") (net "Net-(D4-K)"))
 (segment (start 143.225 93.01) (end 149 98.785) (width 1.5) (layer "B.Cu") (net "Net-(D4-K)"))
 (segment (start 141.46 81.55) (end 141.46 90.47) (width 1.5) (layer "B.Cu") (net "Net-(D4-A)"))
 (segment (start 148.52 74.49) (end 141.46 81.55) (width 1.5) (layer "B.Cu") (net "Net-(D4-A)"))
 (segment (start 149 101.325) (end 149 105.62) (width 1.5) (layer "B.Cu") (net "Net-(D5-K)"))
 (segment (start 149 105.62) (end 149.015 105.635) (width 1.5) (layer "B.Cu") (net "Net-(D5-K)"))
 (segment (start 156.82 74.605) (end 156.82 74.939034) (width 1.5) (layer "B.Cu") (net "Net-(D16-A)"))
 (segment (start 156.82 74.939034) (end 165.765 83.884034) (width 1.5) (layer "B.Cu") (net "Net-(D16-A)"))
 (segment (start 184.74 92.24) (end 184.74 101.905) (width 1.5) (layer "B.Cu") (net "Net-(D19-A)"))
 (segment (start 164.62 74.565) (end 164.695418 74.565) (width 1.5) (layer "B.Cu") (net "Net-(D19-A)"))
 (segment (start 164.695418 74.565) (end 175.130418 85) (width 1.5) (layer "B.Cu") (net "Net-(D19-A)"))
 (segment (start 175.130418 85) (end 177.5 85) (width 1.5) (layer "B.Cu") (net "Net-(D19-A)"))
 (segment (start 177.5 85) (end 184.74 92.24) (width 1.5) (layer "B.Cu") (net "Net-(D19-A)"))
 (segment (start 154.720031 130.860761) (end 160.415 136.55573) (width 1.5) (layer "B.Cu") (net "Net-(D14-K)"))
 (segment (start 154.720031 122.904894) (end 154.720031 130.860761) (width 1.5) (layer "B.Cu") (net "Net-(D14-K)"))
 (segment (start 179.09 106.91) (end 171.5 114.5) (width 1.5) (layer "B.Cu") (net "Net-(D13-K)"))
 (segment (start 160.584925 114.5) (end 154.720031 120.364894) (width 1.5) (layer "B.Cu") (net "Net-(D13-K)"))
 (segment (start 179.09 93.615) (end 179.09 106.91) (width 1.5) (layer "B.Cu") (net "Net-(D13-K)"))
 (segment (start 171.5 114.5) (end 160.584925 114.5) (width 1.5) (layer "B.Cu") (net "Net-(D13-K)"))
 (segment (start 167.77 105.885) (end 168.205 106.32) (width 1.5) (layer "B.Cu") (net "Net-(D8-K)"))
 (segment (start 167.77 101.925) (end 167.77 105.885) (width 1.5) (layer "B.Cu") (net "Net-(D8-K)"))
 (segment (start 173 93.659034) (end 173 109.5) (width 1.5) (layer "B.Cu") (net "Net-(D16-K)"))
 (segment (start 173 109.5) (end 170.5 112) (width 1.5) (layer "B.Cu") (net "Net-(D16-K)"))
 (segment (start 154.524925 112) (end 146.160031 120.364894) (width 1.5) (layer "B.Cu") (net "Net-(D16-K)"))
 (segment (start 170.5 112) (end 154.524925 112) (width 1.5) (layer "B.Cu") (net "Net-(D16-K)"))
 (segment (start 165.765 86.424034) (end 173 93.659034) (width 1.5) (layer "B.Cu") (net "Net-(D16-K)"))
 (segment (start 152.67 74.605) (end 152.67 83.12485) (width 1.5) (layer "B.Cu") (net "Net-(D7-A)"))
 (segment (start 152.67 83.12485) (end 152.495062 83.299788) (width 1.5) (layer "B.Cu") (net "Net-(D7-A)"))
 (segment (start 182.090365 125.655) (end 179.57 125.655) (width 1.5) (layer "B.Cu") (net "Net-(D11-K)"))
 (segment (start 179.57 125.655) (end 171.915 133.31) (width 1.5) (layer "B.Cu") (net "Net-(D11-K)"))
 (segment (start 146.160031 122.904894) (end 146.160031 131.615249) (width 1.5) (layer "B.Cu") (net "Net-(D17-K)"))
 (segment (start 146.160031 131.615249) (end 147.919678 133.374896) (width 1.5) (layer "B.Cu") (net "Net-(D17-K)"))
 (segment (start 163.94 120.35) (end 162.385 120.35) (width 1.5) (layer "B.Cu") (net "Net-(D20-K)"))
 (segment (start 170.24 122.83) (end 166.42 122.83) (width 1.5) (layer "B.Cu") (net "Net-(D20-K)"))
 (segment (start 166.42 122.83) (end 163.94 120.35) (width 1.5) (layer "B.Cu") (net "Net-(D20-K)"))
 (segment (start 184.74 105.79) (end 170.24 120.29) (width 1.5) (layer "B.Cu") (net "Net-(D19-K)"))
 (segment (start 184.74 104.445) (end 184.74 105.79) (width 1.5) (layer "B.Cu") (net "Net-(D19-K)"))
 (segment (start 166.040274 99.385) (end 167.77 99.385) (width 1.5) (layer "B.Cu") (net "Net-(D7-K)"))
 (segment (start 152.495062 85.839788) (end 166.040274 99.385) (width 1.5) (layer "B.Cu") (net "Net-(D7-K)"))
 (segment (start 133.59 121.78) (end 138.6 126.79) (width 1.5) (layer "B.Cu") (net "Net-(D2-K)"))
 (segment (start 133.59 118.294896) (end 133.59 121.78) (width 1.5) (layer "B.Cu") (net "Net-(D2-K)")))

